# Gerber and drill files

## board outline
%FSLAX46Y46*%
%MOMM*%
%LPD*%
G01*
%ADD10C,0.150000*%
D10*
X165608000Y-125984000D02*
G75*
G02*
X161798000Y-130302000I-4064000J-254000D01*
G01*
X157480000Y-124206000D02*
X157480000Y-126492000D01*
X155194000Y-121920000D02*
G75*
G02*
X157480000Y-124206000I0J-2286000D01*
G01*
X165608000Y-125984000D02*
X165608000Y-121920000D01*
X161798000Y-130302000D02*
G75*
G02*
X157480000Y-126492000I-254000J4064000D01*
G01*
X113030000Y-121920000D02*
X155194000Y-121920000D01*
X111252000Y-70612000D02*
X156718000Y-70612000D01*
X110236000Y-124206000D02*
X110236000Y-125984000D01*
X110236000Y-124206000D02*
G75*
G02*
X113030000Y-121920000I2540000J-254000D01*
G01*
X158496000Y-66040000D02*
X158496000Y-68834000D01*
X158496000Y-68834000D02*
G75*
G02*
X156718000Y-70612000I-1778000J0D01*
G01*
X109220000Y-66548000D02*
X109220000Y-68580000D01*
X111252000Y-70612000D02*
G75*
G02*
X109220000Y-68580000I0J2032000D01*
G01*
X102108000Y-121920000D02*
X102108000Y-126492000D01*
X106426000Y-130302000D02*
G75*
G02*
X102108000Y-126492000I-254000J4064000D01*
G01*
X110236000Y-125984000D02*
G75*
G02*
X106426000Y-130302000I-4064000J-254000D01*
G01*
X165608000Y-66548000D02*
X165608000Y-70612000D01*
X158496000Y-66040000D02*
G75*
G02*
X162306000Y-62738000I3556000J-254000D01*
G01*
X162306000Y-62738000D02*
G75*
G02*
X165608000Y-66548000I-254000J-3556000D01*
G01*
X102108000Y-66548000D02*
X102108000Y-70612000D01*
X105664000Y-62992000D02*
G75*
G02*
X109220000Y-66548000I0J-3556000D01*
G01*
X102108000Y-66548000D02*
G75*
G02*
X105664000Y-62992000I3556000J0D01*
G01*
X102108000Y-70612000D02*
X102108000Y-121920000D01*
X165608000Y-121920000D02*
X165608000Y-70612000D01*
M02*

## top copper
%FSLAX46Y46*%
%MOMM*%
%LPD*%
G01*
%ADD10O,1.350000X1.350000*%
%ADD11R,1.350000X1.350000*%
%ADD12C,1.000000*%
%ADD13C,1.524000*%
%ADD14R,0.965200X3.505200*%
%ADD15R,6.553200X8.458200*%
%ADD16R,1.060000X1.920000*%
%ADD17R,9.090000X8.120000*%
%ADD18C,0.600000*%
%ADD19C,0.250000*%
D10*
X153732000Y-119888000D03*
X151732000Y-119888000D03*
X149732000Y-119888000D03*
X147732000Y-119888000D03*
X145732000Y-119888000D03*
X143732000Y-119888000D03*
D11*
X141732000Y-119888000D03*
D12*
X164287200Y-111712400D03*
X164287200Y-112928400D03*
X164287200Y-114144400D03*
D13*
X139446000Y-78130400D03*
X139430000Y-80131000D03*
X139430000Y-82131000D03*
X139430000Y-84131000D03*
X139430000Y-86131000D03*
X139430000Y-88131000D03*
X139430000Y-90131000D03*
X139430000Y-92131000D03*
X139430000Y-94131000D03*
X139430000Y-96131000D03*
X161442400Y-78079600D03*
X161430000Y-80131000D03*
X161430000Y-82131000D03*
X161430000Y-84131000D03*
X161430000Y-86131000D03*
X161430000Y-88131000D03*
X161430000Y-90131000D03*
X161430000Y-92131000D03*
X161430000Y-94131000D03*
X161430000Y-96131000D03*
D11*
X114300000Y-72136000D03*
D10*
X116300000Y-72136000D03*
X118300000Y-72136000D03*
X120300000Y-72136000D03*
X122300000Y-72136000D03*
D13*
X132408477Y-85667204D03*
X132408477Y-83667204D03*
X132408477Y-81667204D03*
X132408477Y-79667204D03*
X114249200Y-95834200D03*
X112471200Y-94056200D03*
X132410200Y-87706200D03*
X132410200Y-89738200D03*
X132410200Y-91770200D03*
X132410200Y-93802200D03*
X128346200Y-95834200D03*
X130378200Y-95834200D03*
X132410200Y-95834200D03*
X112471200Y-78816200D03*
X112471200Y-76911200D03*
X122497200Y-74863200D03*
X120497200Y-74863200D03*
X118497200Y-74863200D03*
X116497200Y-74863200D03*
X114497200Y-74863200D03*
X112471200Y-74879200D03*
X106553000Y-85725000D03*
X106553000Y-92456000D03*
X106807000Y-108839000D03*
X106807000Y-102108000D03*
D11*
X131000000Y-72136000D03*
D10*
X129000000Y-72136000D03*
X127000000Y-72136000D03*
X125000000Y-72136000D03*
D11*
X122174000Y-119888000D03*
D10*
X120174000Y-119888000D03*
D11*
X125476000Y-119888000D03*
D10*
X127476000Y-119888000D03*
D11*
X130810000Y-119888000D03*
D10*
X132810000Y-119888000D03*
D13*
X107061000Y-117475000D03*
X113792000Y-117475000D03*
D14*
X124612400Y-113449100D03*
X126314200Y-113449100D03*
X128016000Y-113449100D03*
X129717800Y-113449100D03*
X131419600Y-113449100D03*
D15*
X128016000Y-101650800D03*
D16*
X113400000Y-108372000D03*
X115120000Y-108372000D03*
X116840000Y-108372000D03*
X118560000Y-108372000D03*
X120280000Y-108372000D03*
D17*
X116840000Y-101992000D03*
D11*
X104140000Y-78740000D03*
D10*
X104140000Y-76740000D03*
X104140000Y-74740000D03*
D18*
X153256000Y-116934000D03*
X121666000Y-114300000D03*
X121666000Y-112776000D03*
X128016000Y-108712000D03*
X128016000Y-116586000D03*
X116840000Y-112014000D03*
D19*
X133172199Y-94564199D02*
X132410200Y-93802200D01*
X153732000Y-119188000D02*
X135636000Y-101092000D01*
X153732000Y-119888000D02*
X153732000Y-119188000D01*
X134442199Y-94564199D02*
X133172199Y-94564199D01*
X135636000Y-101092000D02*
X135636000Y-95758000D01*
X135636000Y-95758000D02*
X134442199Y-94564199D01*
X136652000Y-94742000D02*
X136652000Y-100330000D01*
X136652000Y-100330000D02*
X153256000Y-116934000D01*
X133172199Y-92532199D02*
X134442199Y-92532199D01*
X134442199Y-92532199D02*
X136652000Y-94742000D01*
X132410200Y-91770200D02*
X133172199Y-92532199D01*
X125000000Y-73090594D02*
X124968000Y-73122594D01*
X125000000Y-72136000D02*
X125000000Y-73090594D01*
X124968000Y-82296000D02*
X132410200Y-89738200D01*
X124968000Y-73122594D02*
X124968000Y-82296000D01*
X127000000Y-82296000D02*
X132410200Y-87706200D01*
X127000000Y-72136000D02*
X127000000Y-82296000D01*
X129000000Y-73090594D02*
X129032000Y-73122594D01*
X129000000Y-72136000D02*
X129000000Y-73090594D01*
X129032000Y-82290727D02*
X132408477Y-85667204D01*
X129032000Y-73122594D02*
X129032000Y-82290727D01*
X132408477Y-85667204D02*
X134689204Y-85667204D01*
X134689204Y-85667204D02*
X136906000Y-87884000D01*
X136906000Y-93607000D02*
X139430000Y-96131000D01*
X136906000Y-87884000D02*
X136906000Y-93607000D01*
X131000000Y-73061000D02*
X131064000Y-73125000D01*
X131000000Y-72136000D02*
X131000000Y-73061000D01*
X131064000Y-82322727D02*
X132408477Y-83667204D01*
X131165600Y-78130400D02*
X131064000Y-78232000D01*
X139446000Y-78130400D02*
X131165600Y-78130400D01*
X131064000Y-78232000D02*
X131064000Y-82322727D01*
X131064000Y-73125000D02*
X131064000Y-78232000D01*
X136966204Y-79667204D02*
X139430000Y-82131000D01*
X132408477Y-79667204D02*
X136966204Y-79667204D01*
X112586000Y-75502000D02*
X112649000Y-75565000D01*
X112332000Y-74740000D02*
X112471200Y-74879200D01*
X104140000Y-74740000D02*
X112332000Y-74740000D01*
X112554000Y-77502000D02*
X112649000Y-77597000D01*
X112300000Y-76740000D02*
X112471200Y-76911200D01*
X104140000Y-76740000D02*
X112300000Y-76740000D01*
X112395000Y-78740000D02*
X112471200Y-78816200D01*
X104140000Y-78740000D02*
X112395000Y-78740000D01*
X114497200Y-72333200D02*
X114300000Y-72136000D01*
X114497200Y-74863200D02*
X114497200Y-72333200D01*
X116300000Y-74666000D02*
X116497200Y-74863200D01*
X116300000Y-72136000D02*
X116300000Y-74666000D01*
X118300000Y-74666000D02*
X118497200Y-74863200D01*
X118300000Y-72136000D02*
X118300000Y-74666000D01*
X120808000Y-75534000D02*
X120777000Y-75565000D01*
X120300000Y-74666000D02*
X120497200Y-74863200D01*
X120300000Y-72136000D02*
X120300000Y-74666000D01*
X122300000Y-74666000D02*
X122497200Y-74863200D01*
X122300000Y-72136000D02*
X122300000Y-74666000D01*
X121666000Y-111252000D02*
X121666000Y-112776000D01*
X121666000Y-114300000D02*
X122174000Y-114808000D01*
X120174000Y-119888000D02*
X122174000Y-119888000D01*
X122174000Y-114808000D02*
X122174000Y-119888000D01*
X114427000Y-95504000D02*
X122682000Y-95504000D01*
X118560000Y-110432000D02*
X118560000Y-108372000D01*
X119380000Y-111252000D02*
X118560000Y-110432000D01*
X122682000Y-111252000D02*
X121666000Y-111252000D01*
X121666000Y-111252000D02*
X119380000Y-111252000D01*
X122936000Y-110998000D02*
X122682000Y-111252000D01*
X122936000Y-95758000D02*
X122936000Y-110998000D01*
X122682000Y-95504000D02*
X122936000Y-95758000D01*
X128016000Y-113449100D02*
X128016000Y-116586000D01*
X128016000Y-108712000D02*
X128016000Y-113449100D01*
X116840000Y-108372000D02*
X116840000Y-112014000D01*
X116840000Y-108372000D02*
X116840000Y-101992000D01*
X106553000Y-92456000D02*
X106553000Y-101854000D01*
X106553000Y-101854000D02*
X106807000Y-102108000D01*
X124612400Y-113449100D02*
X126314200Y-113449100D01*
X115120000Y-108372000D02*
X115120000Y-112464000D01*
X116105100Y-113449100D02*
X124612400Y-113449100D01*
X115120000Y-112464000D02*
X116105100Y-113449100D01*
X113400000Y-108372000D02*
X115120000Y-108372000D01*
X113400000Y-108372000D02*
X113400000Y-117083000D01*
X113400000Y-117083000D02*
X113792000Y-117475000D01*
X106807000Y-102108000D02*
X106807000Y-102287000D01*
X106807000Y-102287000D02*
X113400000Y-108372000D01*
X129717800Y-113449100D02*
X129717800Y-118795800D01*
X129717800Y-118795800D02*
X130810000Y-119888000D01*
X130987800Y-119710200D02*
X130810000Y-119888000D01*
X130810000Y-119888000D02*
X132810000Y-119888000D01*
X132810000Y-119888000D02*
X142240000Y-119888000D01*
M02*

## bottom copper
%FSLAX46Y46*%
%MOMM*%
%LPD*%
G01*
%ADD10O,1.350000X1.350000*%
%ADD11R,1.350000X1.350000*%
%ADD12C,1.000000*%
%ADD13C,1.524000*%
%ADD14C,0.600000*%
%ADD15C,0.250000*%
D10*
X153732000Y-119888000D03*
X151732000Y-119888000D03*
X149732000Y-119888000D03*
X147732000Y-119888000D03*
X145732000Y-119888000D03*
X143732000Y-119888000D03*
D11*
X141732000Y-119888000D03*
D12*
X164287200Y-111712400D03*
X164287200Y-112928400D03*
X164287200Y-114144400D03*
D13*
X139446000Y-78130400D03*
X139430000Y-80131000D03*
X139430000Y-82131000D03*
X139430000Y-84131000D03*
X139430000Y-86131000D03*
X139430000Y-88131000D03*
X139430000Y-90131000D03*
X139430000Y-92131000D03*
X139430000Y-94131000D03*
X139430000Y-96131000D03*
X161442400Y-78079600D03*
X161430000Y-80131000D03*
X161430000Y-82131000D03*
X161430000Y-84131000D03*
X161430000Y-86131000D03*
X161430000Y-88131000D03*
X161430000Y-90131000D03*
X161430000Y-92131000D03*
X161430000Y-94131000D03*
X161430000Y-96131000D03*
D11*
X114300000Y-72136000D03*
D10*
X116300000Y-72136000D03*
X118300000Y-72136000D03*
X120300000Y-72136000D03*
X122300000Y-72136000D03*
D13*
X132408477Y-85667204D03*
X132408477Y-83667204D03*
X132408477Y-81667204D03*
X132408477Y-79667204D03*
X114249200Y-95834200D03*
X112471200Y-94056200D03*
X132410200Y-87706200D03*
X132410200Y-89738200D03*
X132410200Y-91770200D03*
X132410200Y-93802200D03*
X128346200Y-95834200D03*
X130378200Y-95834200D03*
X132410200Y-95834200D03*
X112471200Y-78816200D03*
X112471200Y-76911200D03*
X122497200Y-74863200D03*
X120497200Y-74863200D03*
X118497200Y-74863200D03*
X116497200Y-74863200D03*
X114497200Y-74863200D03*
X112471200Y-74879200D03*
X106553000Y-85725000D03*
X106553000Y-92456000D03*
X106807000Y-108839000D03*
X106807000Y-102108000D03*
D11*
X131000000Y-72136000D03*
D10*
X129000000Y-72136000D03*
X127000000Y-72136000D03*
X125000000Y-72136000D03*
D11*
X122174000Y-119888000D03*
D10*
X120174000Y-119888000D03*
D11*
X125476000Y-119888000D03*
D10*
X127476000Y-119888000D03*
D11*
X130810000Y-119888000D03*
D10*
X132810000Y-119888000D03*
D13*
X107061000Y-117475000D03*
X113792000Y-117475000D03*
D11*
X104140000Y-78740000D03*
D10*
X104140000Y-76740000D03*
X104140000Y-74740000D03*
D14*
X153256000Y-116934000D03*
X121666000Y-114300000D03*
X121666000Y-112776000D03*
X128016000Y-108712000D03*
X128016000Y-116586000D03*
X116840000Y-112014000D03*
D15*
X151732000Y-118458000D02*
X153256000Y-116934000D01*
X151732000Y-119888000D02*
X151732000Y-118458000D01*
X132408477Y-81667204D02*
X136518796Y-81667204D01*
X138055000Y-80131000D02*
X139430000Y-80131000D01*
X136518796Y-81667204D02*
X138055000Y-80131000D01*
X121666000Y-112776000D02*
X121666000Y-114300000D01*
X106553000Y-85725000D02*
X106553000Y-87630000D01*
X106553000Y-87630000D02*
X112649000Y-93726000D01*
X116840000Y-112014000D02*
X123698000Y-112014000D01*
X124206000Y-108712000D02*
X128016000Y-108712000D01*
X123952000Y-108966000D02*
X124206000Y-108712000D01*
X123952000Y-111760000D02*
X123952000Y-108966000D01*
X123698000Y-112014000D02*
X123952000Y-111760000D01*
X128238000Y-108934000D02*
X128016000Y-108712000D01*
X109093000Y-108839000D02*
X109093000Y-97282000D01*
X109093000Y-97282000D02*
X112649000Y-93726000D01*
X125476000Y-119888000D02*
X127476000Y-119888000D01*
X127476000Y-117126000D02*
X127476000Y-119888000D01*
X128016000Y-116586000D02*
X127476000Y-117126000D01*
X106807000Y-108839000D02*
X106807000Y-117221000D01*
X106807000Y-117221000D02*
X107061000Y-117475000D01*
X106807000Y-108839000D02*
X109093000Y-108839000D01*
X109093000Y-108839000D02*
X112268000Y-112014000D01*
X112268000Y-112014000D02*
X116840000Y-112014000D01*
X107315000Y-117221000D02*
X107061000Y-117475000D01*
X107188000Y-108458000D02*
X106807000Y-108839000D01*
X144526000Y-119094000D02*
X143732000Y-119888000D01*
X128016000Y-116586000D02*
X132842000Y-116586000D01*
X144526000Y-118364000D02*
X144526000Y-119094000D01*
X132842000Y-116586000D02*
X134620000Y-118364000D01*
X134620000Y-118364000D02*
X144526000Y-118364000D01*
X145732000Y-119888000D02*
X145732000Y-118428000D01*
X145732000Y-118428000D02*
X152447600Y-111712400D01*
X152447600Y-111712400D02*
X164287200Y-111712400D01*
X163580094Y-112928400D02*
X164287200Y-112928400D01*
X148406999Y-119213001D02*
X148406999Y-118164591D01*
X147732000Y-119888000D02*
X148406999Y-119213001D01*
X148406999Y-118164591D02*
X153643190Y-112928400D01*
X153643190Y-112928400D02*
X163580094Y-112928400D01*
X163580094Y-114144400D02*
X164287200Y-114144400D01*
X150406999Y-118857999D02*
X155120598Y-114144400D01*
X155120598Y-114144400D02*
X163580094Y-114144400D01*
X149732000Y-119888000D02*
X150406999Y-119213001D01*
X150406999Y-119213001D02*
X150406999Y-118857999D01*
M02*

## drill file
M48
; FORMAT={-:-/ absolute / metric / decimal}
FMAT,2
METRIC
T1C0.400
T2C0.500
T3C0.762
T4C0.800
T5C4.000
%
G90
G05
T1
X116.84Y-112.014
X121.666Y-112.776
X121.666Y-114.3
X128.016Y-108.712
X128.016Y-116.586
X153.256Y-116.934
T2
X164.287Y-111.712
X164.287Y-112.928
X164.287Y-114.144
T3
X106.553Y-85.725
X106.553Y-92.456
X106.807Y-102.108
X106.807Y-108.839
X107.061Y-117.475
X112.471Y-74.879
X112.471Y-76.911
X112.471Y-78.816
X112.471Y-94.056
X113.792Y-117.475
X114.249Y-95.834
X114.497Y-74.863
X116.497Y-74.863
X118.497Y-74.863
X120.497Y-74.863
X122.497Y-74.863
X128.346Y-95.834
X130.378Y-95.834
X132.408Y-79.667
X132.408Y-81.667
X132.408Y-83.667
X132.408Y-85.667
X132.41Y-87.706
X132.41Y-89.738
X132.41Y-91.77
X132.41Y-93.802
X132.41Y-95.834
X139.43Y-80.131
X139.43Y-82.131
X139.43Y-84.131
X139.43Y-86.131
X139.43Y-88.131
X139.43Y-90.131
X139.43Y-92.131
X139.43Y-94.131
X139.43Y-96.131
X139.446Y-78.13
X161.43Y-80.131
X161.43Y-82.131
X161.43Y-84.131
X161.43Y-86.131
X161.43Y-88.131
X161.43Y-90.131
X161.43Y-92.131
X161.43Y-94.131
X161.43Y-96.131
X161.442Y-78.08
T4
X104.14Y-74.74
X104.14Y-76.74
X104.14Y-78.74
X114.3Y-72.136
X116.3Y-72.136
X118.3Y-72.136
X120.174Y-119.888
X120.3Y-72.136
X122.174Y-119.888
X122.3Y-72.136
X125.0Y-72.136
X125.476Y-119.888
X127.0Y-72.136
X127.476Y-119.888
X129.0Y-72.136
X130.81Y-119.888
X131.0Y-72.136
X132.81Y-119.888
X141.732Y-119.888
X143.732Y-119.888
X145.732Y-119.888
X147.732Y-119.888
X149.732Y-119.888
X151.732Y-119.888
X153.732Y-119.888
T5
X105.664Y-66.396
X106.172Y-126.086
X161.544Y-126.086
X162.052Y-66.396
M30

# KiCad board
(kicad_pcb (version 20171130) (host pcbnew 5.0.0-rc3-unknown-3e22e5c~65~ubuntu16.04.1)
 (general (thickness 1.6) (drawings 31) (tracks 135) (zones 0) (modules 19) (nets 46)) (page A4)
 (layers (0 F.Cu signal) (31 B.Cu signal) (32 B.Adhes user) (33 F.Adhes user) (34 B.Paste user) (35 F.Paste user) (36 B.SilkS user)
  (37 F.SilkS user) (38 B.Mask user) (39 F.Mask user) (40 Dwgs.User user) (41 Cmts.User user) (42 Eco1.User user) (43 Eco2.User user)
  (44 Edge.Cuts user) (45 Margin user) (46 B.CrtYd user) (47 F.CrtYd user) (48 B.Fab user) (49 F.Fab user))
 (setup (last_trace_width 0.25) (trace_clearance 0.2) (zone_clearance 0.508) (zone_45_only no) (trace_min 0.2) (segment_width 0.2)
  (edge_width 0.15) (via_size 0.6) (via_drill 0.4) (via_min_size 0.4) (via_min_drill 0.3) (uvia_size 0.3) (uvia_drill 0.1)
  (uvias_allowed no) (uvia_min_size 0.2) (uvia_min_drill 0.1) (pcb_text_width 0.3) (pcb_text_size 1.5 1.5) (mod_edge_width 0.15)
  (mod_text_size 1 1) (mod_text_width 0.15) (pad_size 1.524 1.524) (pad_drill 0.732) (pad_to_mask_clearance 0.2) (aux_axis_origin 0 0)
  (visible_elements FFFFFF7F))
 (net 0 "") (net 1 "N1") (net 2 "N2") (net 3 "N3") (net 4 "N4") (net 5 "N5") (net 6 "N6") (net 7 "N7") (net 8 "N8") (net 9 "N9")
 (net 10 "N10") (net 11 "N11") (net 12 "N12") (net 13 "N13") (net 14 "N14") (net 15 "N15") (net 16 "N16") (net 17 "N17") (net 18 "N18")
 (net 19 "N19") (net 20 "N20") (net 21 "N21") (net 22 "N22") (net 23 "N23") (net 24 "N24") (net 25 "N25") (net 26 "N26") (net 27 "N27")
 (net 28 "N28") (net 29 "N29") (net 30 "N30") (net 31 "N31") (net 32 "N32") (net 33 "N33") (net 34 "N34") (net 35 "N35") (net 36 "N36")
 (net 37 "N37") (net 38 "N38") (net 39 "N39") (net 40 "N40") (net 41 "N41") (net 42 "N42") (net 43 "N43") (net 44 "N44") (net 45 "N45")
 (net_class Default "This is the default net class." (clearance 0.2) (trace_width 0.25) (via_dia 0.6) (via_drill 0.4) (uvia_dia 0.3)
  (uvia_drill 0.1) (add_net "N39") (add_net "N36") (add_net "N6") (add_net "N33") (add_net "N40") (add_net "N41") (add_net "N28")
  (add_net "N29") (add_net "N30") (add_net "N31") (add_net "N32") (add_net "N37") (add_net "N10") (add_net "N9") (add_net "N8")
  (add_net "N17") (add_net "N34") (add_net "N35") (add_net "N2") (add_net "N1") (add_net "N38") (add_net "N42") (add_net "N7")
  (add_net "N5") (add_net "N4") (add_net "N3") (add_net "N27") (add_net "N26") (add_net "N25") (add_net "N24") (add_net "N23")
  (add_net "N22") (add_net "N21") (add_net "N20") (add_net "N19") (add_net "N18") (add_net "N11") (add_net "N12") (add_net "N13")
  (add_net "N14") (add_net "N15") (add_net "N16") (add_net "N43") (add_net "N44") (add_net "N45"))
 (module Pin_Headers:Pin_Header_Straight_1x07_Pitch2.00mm (layer F.Cu) (at 141.732 119.888 90)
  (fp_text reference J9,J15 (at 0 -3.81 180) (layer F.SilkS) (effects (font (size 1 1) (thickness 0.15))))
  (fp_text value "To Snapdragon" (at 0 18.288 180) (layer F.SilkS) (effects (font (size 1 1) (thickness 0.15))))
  (pad 7 thru_hole oval (at 0 12 90) (size 1.35 1.35) (drill 0.8) (layers *.Cu *.Mask) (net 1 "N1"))
  (pad 6 thru_hole oval (at 0 10 90) (size 1.35 1.35) (drill 0.8) (layers *.Cu *.Mask) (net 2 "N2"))
  (pad 5 thru_hole oval (at 0 8 90) (size 1.35 1.35) (drill 0.8) (layers *.Cu *.Mask) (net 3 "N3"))
  (pad 4 thru_hole oval (at 0 6 90) (size 1.35 1.35) (drill 0.8) (layers *.Cu *.Mask) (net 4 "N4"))
  (pad 3 thru_hole oval (at 0 4 90) (size 1.35 1.35) (drill 0.8) (layers *.Cu *.Mask) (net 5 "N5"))
  (pad 2 thru_hole oval (at 0 2 90) (size 1.35 1.35) (drill 0.8) (layers *.Cu *.Mask) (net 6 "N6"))
  (pad 1 thru_hole rect (at 0 0 90) (size 1.35 1.35) (drill 0.8) (layers *.Cu *.Mask) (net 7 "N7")))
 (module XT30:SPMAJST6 (layer F.Cu) (at 163.576 113.792 270)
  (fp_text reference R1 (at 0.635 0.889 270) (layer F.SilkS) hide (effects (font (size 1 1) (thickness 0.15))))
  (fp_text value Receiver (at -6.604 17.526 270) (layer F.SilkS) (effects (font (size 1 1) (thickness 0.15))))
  (pad 1 thru_hole circle (at -2.0796 -0.7112 270) (size 1 1) (drill 0.5) (layers *.Cu *.Mask) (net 5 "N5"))
  (pad 2 thru_hole circle (at -0.8636 -0.7112 270) (size 1 1) (drill 0.5) (layers *.Cu *.Mask) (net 4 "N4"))
  (pad 3 thru_hole circle (at 0.3524 -0.7112 270) (size 1 1) (drill 0.5) (layers *.Cu *.Mask) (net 3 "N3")))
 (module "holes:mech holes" (layer F.Cu) (at 162.052 129.286)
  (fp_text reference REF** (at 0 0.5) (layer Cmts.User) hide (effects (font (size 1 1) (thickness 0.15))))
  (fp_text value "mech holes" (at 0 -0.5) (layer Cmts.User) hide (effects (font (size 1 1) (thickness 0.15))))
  (pad "" np_thru_hole circle (at -0.508 -3.2004) (size 4 4) (drill 4) (layers *.Cu *.Mask)))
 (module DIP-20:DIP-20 (layer F.Cu) (at 138.176 104.14)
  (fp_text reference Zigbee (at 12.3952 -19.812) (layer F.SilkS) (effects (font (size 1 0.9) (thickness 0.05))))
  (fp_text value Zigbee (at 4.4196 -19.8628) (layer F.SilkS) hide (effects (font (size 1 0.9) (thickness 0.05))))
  (pad 1 thru_hole circle (at 1.27 -26.0096) (size 1.524 1.524) (drill 0.762) (layers *.Cu *.Mask F.SilkS) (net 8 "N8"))
  (pad 2 thru_hole circle (at 1.254 -24.009) (size 1.524 1.524) (drill 0.762) (layers *.Cu *.Mask F.SilkS) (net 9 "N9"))
  (pad 3 thru_hole circle (at 1.254 -22.009) (size 1.524 1.524) (drill 0.762) (layers *.Cu *.Mask F.SilkS) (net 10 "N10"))
  (pad 4 thru_hole circle (at 1.254 -20.009) (size 1.524 1.524) (drill 0.762) (layers *.Cu *.Mask F.SilkS) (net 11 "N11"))
  (pad 5 thru_hole circle (at 1.254 -18.009) (size 1.524 1.524) (drill 0.762) (layers *.Cu *.Mask F.SilkS) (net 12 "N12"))
  (pad 6 thru_hole circle (at 1.254 -16.009) (size 1.524 1.524) (drill 0.762) (layers *.Cu *.Mask F.SilkS) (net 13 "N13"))
  (pad 7 thru_hole circle (at 1.254 -14.009) (size 1.524 1.524) (drill 0.762) (layers *.Cu *.Mask F.SilkS) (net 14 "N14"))
  (pad 8 thru_hole circle (at 1.254 -12.009) (size 1.524 1.524) (drill 0.762) (layers *.Cu *.Mask F.SilkS) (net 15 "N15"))
  (pad 9 thru_hole circle (at 1.254 -10.009) (size 1.524 1.524) (drill 0.762) (layers *.Cu *.Mask F.SilkS) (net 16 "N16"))
  (pad 10 thru_hole circle (at 1.254 -8.009) (size 1.524 1.524) (drill 0.762) (layers *.Cu *.Mask F.SilkS) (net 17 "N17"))
  (pad 20 thru_hole circle (at 23.2664 -26.0604) (size 1.524 1.524) (drill 0.762) (layers *.Cu *.Mask F.SilkS) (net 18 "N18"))
  (pad 19 thru_hole circle (at 23.254 -24.009) (size 1.524 1.524) (drill 0.762) (layers *.Cu *.Mask F.SilkS) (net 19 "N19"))
  (pad 18 thru_hole circle (at 23.254 -22.009) (size 1.524 1.524) (drill 0.762) (layers *.Cu *.Mask F.SilkS) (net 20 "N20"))
  (pad 17 thru_hole circle (at 23.254 -20.009) (size 1.524 1.524) (drill 0.762) (layers *.Cu *.Mask F.SilkS) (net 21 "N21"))
  (pad 16 thru_hole circle (at 23.254 -18.009) (size 1.524 1.524) (drill 0.762) (layers *.Cu *.Mask F.SilkS) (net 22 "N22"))
  (pad 15 thru_hole circle (at 23.254 -16.009) (size 1.524 1.524) (drill 0.762) (layers *.Cu *.Mask F.SilkS) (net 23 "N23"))
  (pad 14 thru_hole circle (at 23.254 -14.009) (size 1.524 1.524) (drill 0.762) (layers *.Cu *.Mask F.SilkS) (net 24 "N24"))
  (pad 13 thru_hole circle (at 23.254 -12.009) (size 1.524 1.524) (drill 0.762) (layers *.Cu *.Mask F.SilkS) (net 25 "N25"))
  (pad 12 thru_hole circle (at 23.254 -10.009) (size 1.524 1.524) (drill 0.762) (layers *.Cu *.Mask F.SilkS) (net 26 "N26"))
  (pad 11 thru_hole circle (at 23.254 -8.009) (size 1.524 1.524) (drill 0.762) (layers *.Cu *.Mask F.SilkS) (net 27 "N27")))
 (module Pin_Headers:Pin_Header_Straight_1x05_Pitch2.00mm (layer F.Cu) (at 114.3 72.136 90)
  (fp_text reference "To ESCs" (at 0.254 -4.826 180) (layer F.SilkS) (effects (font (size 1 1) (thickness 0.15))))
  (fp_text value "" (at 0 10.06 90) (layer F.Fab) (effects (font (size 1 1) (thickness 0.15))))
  (pad 1 thru_hole rect (at 0 0 90) (size 1.35 1.35) (drill 0.8) (layers *.Cu *.Mask) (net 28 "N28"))
  (pad 2 thru_hole oval (at 0 2 90) (size 1.35 1.35) (drill 0.8) (layers *.Cu *.Mask) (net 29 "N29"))
  (pad 3 thru_hole oval (at 0 4 90) (size 1.35 1.35) (drill 0.8) (layers *.Cu *.Mask) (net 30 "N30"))
  (pad 4 thru_hole oval (at 0 6 90) (size 1.35 1.35) (drill 0.8) (layers *.Cu *.Mask) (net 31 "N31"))
  (pad 5 thru_hole oval (at 0 8 90) (size 1.35 1.35) (drill 0.8) (layers *.Cu *.Mask) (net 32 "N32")))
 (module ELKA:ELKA (layer F.Cu) (at 121.666 85.852)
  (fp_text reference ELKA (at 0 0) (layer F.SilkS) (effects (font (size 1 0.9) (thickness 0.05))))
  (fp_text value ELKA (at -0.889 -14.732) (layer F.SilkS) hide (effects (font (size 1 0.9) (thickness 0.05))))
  (pad D thru_hole circle (at 10.742477 -0.184796) (size 1.524 1.524) (drill 0.762) (layers *.Cu *.Mask B.SilkS) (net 17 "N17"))
  (pad C thru_hole circle (at 10.742477 -2.184796) (size 1.524 1.524) (drill 0.762) (layers *.Cu *.Mask B.SilkS) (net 8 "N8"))
  (pad B thru_hole circle (at 10.742477 -4.184796) (size 1.524 1.524) (drill 0.762) (layers *.Cu *.Mask B.SilkS) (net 9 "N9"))
  (pad A thru_hole circle (at 10.742477 -6.184796) (size 1.524 1.524) (drill 0.762) (layers *.Cu *.Mask B.SilkS) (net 10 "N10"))
  (pad 12 thru_hole circle (at -7.4168 9.9822) (size 1.524 1.524) (drill 0.762) (layers *.Cu *.Mask B.SilkS) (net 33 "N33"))
  (pad 11 thru_hole circle (at -9.1948 8.2042 270) (size 1.524 1.524) (drill 0.762) (layers *.Cu *.Mask B.SilkS) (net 6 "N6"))
  (pad E thru_hole circle (at 10.7442 1.8542 270) (size 1.524 1.524) (drill 0.762) (layers *.Cu *.Mask B.SilkS) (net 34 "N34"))
  (pad F thru_hole circle (at 10.7442 3.8862 270) (size 1.524 1.524) (drill 0.762) (layers *.Cu *.Mask B.SilkS) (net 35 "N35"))
  (pad G thru_hole circle (at 10.7442 5.9182 270) (size 1.524 1.524) (drill 0.762) (layers *.Cu *.Mask B.SilkS) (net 2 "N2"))
  (pad H thru_hole circle (at 10.7442 7.9502 270) (size 1.524 1.524) (drill 0.762) (layers *.Cu *.Mask B.SilkS) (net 1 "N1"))
  (pad 10 thru_hole circle (at 6.6802 9.9822 270) (size 1.524 1.524) (drill 0.762) (layers *.Cu *.Mask B.SilkS) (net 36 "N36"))
  (pad 9 thru_hole circle (at 8.7122 9.9822 270) (size 1.524 1.524) (drill 0.762) (layers *.Cu *.Mask B.SilkS) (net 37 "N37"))
  (pad I thru_hole circle (at 10.7442 9.9822 270) (size 1.524 1.524) (drill 0.762) (layers *.Cu *.Mask B.SilkS) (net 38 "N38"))
  (pad 1 thru_hole circle (at -9.1948 -7.0358 270) (size 1.524 1.524) (drill 0.762) (layers *.Cu *.Mask B.SilkS) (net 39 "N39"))
  (pad 2 thru_hole circle (at -9.1948 -8.9408 270) (size 1.524 1.524) (drill 0.762) (layers *.Cu *.Mask B.SilkS) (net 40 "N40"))
  (pad 8 thru_hole circle (at 0.8312 -10.9888 270) (size 1.524 1.524) (drill 0.762) (layers *.Cu *.Mask B.SilkS) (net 32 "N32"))
  (pad 7 thru_hole circle (at -1.1688 -10.9888 270) (size 1.524 1.524) (drill 0.762) (layers *.Cu *.Mask B.SilkS) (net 31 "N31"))
  (pad 6 thru_hole circle (at -3.1688 -10.9888 270) (size 1.524 1.524) (drill 0.762) (layers *.Cu *.Mask B.SilkS) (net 30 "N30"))
  (pad 5 thru_hole circle (at -5.1688 -10.9888 270) (size 1.524 1.524) (drill 0.762) (layers *.Cu *.Mask B.SilkS) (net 29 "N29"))
  (pad 4 thru_hole circle (at -7.1688 -10.9888 270) (size 1.524 1.524) (drill 0.762) (layers *.Cu *.Mask B.SilkS) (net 28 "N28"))
  (pad 3 thru_hole circle (at -9.1948 -10.9728 270) (size 1.524 1.524) (drill 0.762) (layers *.Cu *.Mask B.SilkS) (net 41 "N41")))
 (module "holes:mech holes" (layer F.Cu) (at 106.172 69.596)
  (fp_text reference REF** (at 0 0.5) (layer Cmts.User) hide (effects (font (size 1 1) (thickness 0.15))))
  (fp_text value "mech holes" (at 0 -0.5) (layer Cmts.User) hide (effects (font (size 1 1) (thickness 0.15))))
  (pad "" np_thru_hole circle (at -0.508 -3.2004) (size 4 4) (drill 4) (layers *.Cu *.Mask)))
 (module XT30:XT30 (layer F.Cu) (at 112.522 87.122 270)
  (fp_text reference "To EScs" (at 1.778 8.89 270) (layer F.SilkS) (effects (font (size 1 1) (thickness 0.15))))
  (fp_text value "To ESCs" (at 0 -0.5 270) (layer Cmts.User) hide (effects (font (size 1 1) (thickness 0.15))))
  (pad 1 thru_hole circle (at -1.397 5.969 270) (size 1.524 1.524) (drill 0.762) (layers *.Cu *.Mask) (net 6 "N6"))
  (pad 2 thru_hole circle (at 5.334 5.969 270) (size 1.524 1.524) (drill 0.762) (layers *.Cu *.Mask) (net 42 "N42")))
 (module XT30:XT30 (layer F.Cu) (at 100.838 107.442 90)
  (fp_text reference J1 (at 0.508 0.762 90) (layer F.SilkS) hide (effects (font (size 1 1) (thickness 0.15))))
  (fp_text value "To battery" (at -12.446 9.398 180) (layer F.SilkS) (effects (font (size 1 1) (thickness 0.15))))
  (pad 1 thru_hole circle (at -1.397 5.969 90) (size 1.524 1.524) (drill 0.762) (layers *.Cu *.Mask) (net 6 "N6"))
  (pad 2 thru_hole circle (at 5.334 5.969 90) (size 1.524 1.524) (drill 0.762) (layers *.Cu *.Mask) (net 42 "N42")))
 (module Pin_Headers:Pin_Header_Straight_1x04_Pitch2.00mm (layer F.Cu) (at 131 72.136 270)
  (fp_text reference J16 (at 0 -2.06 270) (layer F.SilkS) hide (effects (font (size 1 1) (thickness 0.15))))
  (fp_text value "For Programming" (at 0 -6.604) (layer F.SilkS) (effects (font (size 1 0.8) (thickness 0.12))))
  (pad 1 thru_hole rect (at 0 0 270) (size 1.35 1.35) (drill 0.8) (layers *.Cu *.Mask) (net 8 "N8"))
  (pad 2 thru_hole oval (at 0 2 270) (size 1.35 1.35) (drill 0.8) (layers *.Cu *.Mask) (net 17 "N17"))
  (pad 3 thru_hole oval (at 0 4 270) (size 1.35 1.35) (drill 0.8) (layers *.Cu *.Mask) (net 34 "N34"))
  (pad 4 thru_hole oval (at 0 6 270) (size 1.35 1.35) (drill 0.8) (layers *.Cu *.Mask) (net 35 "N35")))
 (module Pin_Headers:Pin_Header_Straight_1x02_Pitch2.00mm (layer F.Cu) (at 122.174 119.888 270)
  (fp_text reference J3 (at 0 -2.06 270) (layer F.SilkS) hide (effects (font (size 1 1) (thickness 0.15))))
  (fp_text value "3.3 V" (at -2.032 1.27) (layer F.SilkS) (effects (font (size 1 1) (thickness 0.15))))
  (pad 1 thru_hole rect (at 0 0 270) (size 1.35 1.35) (drill 0.8) (layers *.Cu *.Mask) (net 33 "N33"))
  (pad 2 thru_hole oval (at 0 2 270) (size 1.35 1.35) (drill 0.8) (layers *.Cu *.Mask) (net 33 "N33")))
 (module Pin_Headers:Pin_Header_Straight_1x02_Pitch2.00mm (layer F.Cu) (at 125.476 119.888 90)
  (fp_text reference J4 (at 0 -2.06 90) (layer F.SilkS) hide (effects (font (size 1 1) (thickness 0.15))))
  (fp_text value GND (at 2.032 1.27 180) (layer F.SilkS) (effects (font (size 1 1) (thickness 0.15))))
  (pad 1 thru_hole rect (at 0 0 90) (size 1.35 1.35) (drill 0.8) (layers *.Cu *.Mask) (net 6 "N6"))
  (pad 2 thru_hole oval (at 0 2 90) (size 1.35 1.35) (drill 0.8) (layers *.Cu *.Mask) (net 6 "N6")))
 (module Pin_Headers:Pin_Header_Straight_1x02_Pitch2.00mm (layer F.Cu) (at 130.81 119.888 90)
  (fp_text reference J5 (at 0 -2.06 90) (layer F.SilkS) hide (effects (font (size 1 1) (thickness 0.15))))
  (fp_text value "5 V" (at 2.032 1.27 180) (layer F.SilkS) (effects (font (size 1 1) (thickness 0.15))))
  (pad 1 thru_hole rect (at 0 0 90) (size 1.35 1.35) (drill 0.8) (layers *.Cu *.Mask) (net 7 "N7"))
  (pad 2 thru_hole oval (at 0 2 90) (size 1.35 1.35) (drill 0.8) (layers *.Cu *.Mask) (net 7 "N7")))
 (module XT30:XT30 (layer F.Cu) (at 108.458 111.506)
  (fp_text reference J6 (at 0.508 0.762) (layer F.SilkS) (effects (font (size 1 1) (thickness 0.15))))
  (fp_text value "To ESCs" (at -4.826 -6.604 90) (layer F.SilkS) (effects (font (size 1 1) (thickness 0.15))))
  (pad 1 thru_hole circle (at -1.397 5.969) (size 1.524 1.524) (drill 0.762) (layers *.Cu *.Mask) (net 6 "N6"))
  (pad 2 thru_hole circle (at 5.334 5.969) (size 1.524 1.524) (drill 0.762) (layers *.Cu *.Mask) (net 42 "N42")))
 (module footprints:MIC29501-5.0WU (layer F.Cu) (at 128.016 104.394)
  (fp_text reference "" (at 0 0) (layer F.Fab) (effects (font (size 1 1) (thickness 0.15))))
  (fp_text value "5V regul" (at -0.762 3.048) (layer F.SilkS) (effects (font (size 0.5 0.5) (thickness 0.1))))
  (pad 1 smd rect (at -3.4036 9.0551) (size 0.9652 3.5052) (layers F.Cu F.Paste F.Mask) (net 42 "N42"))
  (pad 2 smd rect (at -1.7018 9.0551) (size 0.9652 3.5052) (layers F.Cu F.Paste F.Mask) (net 42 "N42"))
  (pad 3 smd rect (at 0 9.0551) (size 0.9652 3.5052) (layers F.Cu F.Paste F.Mask) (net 6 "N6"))
  (pad 4 smd rect (at 1.7018 9.0551) (size 0.9652 3.5052) (layers F.Cu F.Paste F.Mask) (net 7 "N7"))
  (pad 5 smd rect (at 3.4036 9.0551) (size 0.9652 3.5052) (layers F.Cu F.Paste F.Mask) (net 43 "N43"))
  (pad 6 smd rect (at 0 -2.7432) (size 6.5532 8.4582) (layers F.Cu F.Paste F.Mask) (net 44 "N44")))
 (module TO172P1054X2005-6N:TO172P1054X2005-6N (layer F.Cu) (at 116.84 103.632)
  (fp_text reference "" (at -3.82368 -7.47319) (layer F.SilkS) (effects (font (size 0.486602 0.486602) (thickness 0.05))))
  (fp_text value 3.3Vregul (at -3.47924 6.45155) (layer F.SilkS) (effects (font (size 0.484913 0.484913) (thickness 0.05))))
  (pad 1 smd rect (at -3.44 4.74 90) (size 1.92 1.06) (layers F.Cu F.Paste F.Mask) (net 42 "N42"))
  (pad 2 smd rect (at -1.72 4.74 90) (size 1.92 1.06) (layers F.Cu F.Paste F.Mask) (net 42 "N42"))
  (pad 3 smd rect (at 0 4.74 90) (size 1.92 1.06) (layers F.Cu F.Paste F.Mask) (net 6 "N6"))
  (pad 4 smd rect (at 1.72 4.74 90) (size 1.92 1.06) (layers F.Cu F.Paste F.Mask) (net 33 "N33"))
  (pad 5 smd rect (at 3.44 4.74 90) (size 1.92 1.06) (layers F.Cu F.Paste F.Mask) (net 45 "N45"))
  (pad 6 smd rect (at 0 -1.64 90) (size 8.12 9.09) (layers F.Cu F.Paste F.Mask) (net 6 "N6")))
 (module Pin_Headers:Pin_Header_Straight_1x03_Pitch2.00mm (layer F.Cu) (at 104.14 78.74 180)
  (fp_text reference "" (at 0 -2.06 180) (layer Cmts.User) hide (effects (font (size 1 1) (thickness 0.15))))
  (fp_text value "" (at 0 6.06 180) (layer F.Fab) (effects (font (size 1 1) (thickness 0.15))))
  (pad 1 thru_hole rect (at 0 0 180) (size 1.35 1.35) (drill 0.8) (layers *.Cu *.Mask) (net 39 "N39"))
  (pad 2 thru_hole oval (at 0 2 180) (size 1.35 1.35) (drill 0.8) (layers *.Cu *.Mask) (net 40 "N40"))
  (pad 3 thru_hole oval (at 0 4 180) (size 1.35 1.35) (drill 0.8) (layers *.Cu *.Mask) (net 41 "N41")))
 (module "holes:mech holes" (layer F.Cu) (at 162.56 69.596)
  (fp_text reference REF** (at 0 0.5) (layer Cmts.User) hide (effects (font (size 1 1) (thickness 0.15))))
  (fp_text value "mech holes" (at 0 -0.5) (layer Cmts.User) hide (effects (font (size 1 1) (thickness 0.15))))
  (pad "" np_thru_hole circle (at -0.508 -3.2004) (size 4 4) (drill 4) (layers *.Cu *.Mask)))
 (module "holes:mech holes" (layer F.Cu) (at 106.68 129.286)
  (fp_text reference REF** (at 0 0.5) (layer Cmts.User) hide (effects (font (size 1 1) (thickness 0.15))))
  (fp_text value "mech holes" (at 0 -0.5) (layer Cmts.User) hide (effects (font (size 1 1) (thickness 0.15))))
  (pad "" np_thru_hole circle (at -0.508 -3.2004) (size 4 4) (drill 4) (layers *.Cu *.Mask)))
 (gr_arc (start 161.544 126.238) (end 165.608 125.984) (angle 90) (layer Edge.Cuts) (width 0.15))
 (gr_line (start 157.48 124.206) (end 157.48 126.492) (angle 90) (layer Edge.Cuts) (width 0.15))
 (gr_arc (start 155.194 124.206) (end 155.194 121.92) (angle 90) (layer Edge.Cuts) (width 0.15))
 (gr_line (start 165.608 125.984) (end 165.608 121.92) (angle 90) (layer Edge.Cuts) (width 0.15))
 (gr_arc (start 161.544 126.238) (end 161.798 130.302) (angle 90) (layer Edge.Cuts) (width 0.15))
 (gr_line (start 113.03 121.92) (end 155.194 121.92) (angle 90) (layer Edge.Cuts) (width 0.15))
 (gr_line (start 111.252 70.612) (end 156.718 70.612) (angle 90) (layer Edge.Cuts) (width 0.15))
 (gr_line (start 110.236 124.206) (end 110.236 125.984) (angle 90) (layer Edge.Cuts) (width 0.15))
 (gr_arc (start 112.776 124.46) (end 110.236 124.206) (angle 90) (layer Edge.Cuts) (width 0.15))
 (gr_line (start 158.496 66.04) (end 158.496 68.834) (angle 90) (layer Edge.Cuts) (width 0.15))
 (gr_arc (start 156.718 68.834) (end 158.496 68.834) (angle 90) (layer Edge.Cuts) (width 0.15))
 (gr_line (start 109.22 66.548) (end 109.22 68.58) (angle 90) (layer Edge.Cuts) (width 0.15))
 (gr_arc (start 111.252 68.58) (end 111.252 70.612) (angle 90) (layer Edge.Cuts) (width 0.15))
 (gr_line (start 102.108 121.92) (end 102.108 126.492) (angle 90) (layer Edge.Cuts) (width 0.15))
 (gr_arc (start 106.172 126.238) (end 106.426 130.302) (angle 90) (layer Edge.Cuts) (width 0.15))
 (gr_arc (start 106.172 126.238) (end 110.236 125.984) (angle 90) (layer Edge.Cuts) (width 0.15))
 (gr_line (start 165.608 66.548) (end 165.608 70.612) (angle 90) (layer Edge.Cuts) (width 0.15))
 (gr_arc (start 162.052 66.294) (end 158.496 66.04) (angle 90) (layer Edge.Cuts) (width 0.15))
 (gr_arc (start 162.052 66.294) (end 162.306 62.738) (angle 90) (layer Edge.Cuts) (width 0.15))
 (gr_line (start 102.108 66.548) (end 102.108 70.612) (angle 90) (layer Edge.Cuts) (width 0.15))
 (gr_arc (start 105.664 66.548) (end 105.664 62.992) (angle 90) (layer Edge.Cuts) (width 0.15))
 (gr_arc (start 105.664 66.548) (end 102.108 66.548) (angle 90) (layer Edge.Cuts) (width 0.15))
 (gr_line (start 102.108 70.612) (end 102.108 121.92) (angle 90) (layer Edge.Cuts) (width 0.15))
 (gr_line (start 165.608 121.92) (end 165.608 70.612) (angle 90) (layer Edge.Cuts) (width 0.15))
 (segment (start 133.172199 94.564199) (end 132.4102 93.8022) (width 0.25) (layer F.Cu) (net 1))
 (segment (start 153.732 119.188) (end 135.636 101.092) (width 0.25) (layer F.Cu) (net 1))
 (segment (start 153.732 119.888) (end 153.732 119.188) (width 0.25) (layer F.Cu) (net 1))
 (segment (start 134.442199 94.564199) (end 133.172199 94.564199) (width 0.25) (layer F.Cu) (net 1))
 (segment (start 135.636 101.092) (end 135.636 95.758) (width 0.25) (layer F.Cu) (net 1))
 (segment (start 135.636 95.758) (end 134.442199 94.564199) (width 0.25) (layer F.Cu) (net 1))
 (segment (start 136.652 94.742) (end 136.652 100.33) (width 0.25) (layer F.Cu) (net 2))
 (segment (start 136.652 100.33) (end 153.256 116.934) (width 0.25) (layer F.Cu) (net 2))
 (segment (start 133.172199 92.532199) (end 134.442199 92.532199) (width 0.25) (layer F.Cu) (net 2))
 (segment (start 134.442199 92.532199) (end 136.652 94.742) (width 0.25) (layer F.Cu) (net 2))
 (segment (start 132.4102 91.7702) (end 133.172199 92.532199) (width 0.25) (layer F.Cu) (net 2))
 (via (at 153.256 116.934) (size 0.6) (drill 0.4) (layers F.Cu B.Cu) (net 2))
 (segment (start 151.732 118.458) (end 153.256 116.934) (width 0.25) (layer B.Cu) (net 2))
 (segment (start 151.732 119.888) (end 151.732 118.458) (width 0.25) (layer B.Cu) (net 2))
 (segment (start 125 73.090594) (end 124.968 73.122594) (width 0.25) (layer F.Cu) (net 35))
 (segment (start 125 72.136) (end 125 73.090594) (width 0.25) (layer F.Cu) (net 35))
 (segment (start 124.968 82.296) (end 132.4102 89.7382) (width 0.25) (layer F.Cu) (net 35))
 (segment (start 124.968 73.122594) (end 124.968 82.296) (width 0.25) (layer F.Cu) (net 35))
 (segment (start 127 82.296) (end 132.4102 87.7062) (width 0.25) (layer F.Cu) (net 34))
 (segment (start 127 72.136) (end 127 82.296) (width 0.25) (layer F.Cu) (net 34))
 (segment (start 129 73.090594) (end 129.032 73.122594) (width 0.25) (layer F.Cu) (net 17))
 (segment (start 129 72.136) (end 129 73.090594) (width 0.25) (layer F.Cu) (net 17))
 (segment (start 129.032 82.290727) (end 132.408477 85.667204) (width 0.25) (layer F.Cu) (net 17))
 (segment (start 129.032 73.122594) (end 129.032 82.290727) (width 0.25) (layer F.Cu) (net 17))
 (segment (start 132.408477 85.667204) (end 134.689204 85.667204) (width 0.25) (layer F.Cu) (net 17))
 (segment (start 134.689204 85.667204) (end 136.906 87.884) (width 0.25) (layer F.Cu) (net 17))
 (segment (start 136.906 93.607) (end 139.43 96.131) (width 0.25) (layer F.Cu) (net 17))
 (segment (start 136.906 87.884) (end 136.906 93.607) (width 0.25) (layer F.Cu) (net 17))
 (segment (start 131 73.061) (end 131.064 73.125) (width 0.25) (layer F.Cu) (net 8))
 (segment (start 131 72.136) (end 131 73.061) (width 0.25) (layer F.Cu) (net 8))
 (segment (start 131.064 82.322727) (end 132.408477 83.667204) (width 0.25) (layer F.Cu) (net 8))
 (segment (start 131.1656 78.1304) (end 131.064 78.232) (width 0.25) (layer F.Cu) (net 8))
 (segment (start 139.446 78.1304) (end 131.1656 78.1304) (width 0.25) (layer F.Cu) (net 8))
 (segment (start 131.064 78.232) (end 131.064 82.322727) (width 0.25) (layer F.Cu) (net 8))
 (segment (start 131.064 73.125) (end 131.064 78.232) (width 0.25) (layer F.Cu) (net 8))
 (segment (start 132.408477 81.667204) (end 136.518796 81.667204) (width 0.25) (layer B.Cu) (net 9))
 (segment (start 138.055 80.131) (end 139.43 80.131) (width 0.25) (layer B.Cu) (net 9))
 (segment (start 136.518796 81.667204) (end 138.055 80.131) (width 0.25) (layer B.Cu) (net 9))
 (segment (start 136.966204 79.667204) (end 139.43 82.131) (width 0.25) (layer F.Cu) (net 10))
 (segment (start 132.408477 79.667204) (end 136.966204 79.667204) (width 0.25) (layer F.Cu) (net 10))
 (segment (start 112.586 75.502) (end 112.649 75.565) (width 0.25) (layer F.Cu) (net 41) (status 30))
 (segment (start 112.332 74.74) (end 112.4712 74.8792) (width 0.25) (layer F.Cu) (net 41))
 (segment (start 104.14 74.74) (end 112.332 74.74) (width 0.25) (layer F.Cu) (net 41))
 (segment (start 112.554 77.502) (end 112.649 77.597) (width 0.25) (layer F.Cu) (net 40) (status 30))
 (segment (start 112.3 76.74) (end 112.4712 76.9112) (width 0.25) (layer F.Cu) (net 40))
 (segment (start 104.14 76.74) (end 112.3 76.74) (width 0.25) (layer F.Cu) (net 40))
 (segment (start 112.395 78.74) (end 112.4712 78.8162) (width 0.25) (layer F.Cu) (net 39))
 (segment (start 104.14 78.74) (end 112.395 78.74) (width 0.25) (layer F.Cu) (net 39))
 (segment (start 114.4972 72.3332) (end 114.3 72.136) (width 0.25) (layer F.Cu) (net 28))
 (segment (start 114.4972 74.8632) (end 114.4972 72.3332) (width 0.25) (layer F.Cu) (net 28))
 (segment (start 116.3 74.666) (end 116.4972 74.8632) (width 0.25) (layer F.Cu) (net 29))
 (segment (start 116.3 72.136) (end 116.3 74.666) (width 0.25) (layer F.Cu) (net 29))
 (segment (start 118.3 74.666) (end 118.4972 74.8632) (width 0.25) (layer F.Cu) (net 30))
 (segment (start 118.3 72.136) (end 118.3 74.666) (width 0.25) (layer F.Cu) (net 30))
 (segment (start 120.808 75.534) (end 120.777 75.565) (width 0.25) (layer F.Cu) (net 31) (status 30))
 (segment (start 120.3 74.666) (end 120.4972 74.8632) (width 0.25) (layer F.Cu) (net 31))
 (segment (start 120.3 72.136) (end 120.3 74.666) (width 0.25) (layer F.Cu) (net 31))
 (segment (start 122.3 74.666) (end 122.4972 74.8632) (width 0.25) (layer F.Cu) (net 32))
 (segment (start 122.3 72.136) (end 122.3 74.666) (width 0.25) (layer F.Cu) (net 32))
 (segment (start 121.666 111.252) (end 121.666 112.776) (width 0.25) (layer F.Cu) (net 33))
 (segment (start 121.666 114.3) (end 122.174 114.808) (width 0.25) (layer F.Cu) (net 33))
 (via (at 121.666 114.3) (size 0.6) (drill 0.4) (layers F.Cu B.Cu) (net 33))
 (segment (start 121.666 112.776) (end 121.666 114.3) (width 0.25) (layer B.Cu) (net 33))
 (via (at 121.666 112.776) (size 0.6) (drill 0.4) (layers F.Cu B.Cu) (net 33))
 (segment (start 120.174 119.888) (end 122.174 119.888) (width 0.25) (layer F.Cu) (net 33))
 (segment (start 122.174 114.808) (end 122.174 119.888) (width 0.25) (layer F.Cu) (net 33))
 (segment (start 114.427 95.504) (end 122.682 95.504) (width 0.25) (layer F.Cu) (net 33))
 (segment (start 118.56 110.432) (end 118.56 108.372) (width 0.25) (layer F.Cu) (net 33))
 (segment (start 119.38 111.252) (end 118.56 110.432) (width 0.25) (layer F.Cu) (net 33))
 (segment (start 122.682 111.252) (end 121.666 111.252) (width 0.25) (layer F.Cu) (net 33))
 (segment (start 121.666 111.252) (end 119.38 111.252) (width 0.25) (layer F.Cu) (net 33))
 (segment (start 122.936 110.998) (end 122.682 111.252) (width 0.25) (layer F.Cu) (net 33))
 (segment (start 122.936 95.758) (end 122.936 110.998) (width 0.25) (layer F.Cu) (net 33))
 (segment (start 122.682 95.504) (end 122.936 95.758) (width 0.25) (layer F.Cu) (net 33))
 (segment (start 106.553 85.725) (end 106.553 87.63) (width 0.25) (layer B.Cu) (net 6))
 (segment (start 106.553 87.63) (end 112.649 93.726) (width 0.25) (layer B.Cu) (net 6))
 (segment (start 116.84 112.014) (end 123.698 112.014) (width 0.25) (layer B.Cu) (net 6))
 (segment (start 124.206 108.712) (end 128.016 108.712) (width 0.25) (layer B.Cu) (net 6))
 (segment (start 123.952 108.966) (end 124.206 108.712) (width 0.25) (layer B.Cu) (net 6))
 (segment (start 123.952 111.76) (end 123.952 108.966) (width 0.25) (layer B.Cu) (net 6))
 (segment (start 123.698 112.014) (end 123.952 111.76) (width 0.25) (layer B.Cu) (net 6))
 (segment (start 128.238 108.934) (end 128.016 108.712) (width 0.25) (layer B.Cu) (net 6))
 (via (at 128.016 108.712) (size 0.6) (drill 0.4) (layers F.Cu B.Cu) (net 6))
 (segment (start 109.093 108.839) (end 109.093 97.282) (width 0.25) (layer B.Cu) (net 6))
 (segment (start 109.093 97.282) (end 112.649 93.726) (width 0.25) (layer B.Cu) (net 6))
 (segment (start 125.476 119.888) (end 127.476 119.888) (width 0.25) (layer B.Cu) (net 6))
 (segment (start 128.016 113.4491) (end 128.016 116.586) (width 0.25) (layer F.Cu) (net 6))
 (segment (start 127.476 117.126) (end 127.476 119.888) (width 0.25) (layer B.Cu) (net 6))
 (segment (start 128.016 116.586) (end 127.476 117.126) (width 0.25) (layer B.Cu) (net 6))
 (via (at 128.016 116.586) (size 0.6) (drill 0.4) (layers F.Cu B.Cu) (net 6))
 (segment (start 106.807 108.839) (end 106.807 117.221) (width 0.25) (layer B.Cu) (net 6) (status 10))
 (segment (start 106.807 117.221) (end 107.061 117.475) (width 0.25) (layer B.Cu) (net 6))
 (segment (start 128.016 108.712) (end 128.016 113.4491) (width 0.25) (layer F.Cu) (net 6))
 (segment (start 116.84 108.372) (end 116.84 112.014) (width 0.25) (layer F.Cu) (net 6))
 (via (at 116.84 112.014) (size 0.6) (drill 0.4) (layers F.Cu B.Cu) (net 6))
 (segment (start 106.807 108.839) (end 109.093 108.839) (width 0.25) (layer B.Cu) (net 6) (status 10))
 (segment (start 109.093 108.839) (end 112.268 112.014) (width 0.25) (layer B.Cu) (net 6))
 (segment (start 112.268 112.014) (end 116.84 112.014) (width 0.25) (layer B.Cu) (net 6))
 (segment (start 107.315 117.221) (end 107.061 117.475) (width 0.25) (layer B.Cu) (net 6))
 (segment (start 107.188 108.458) (end 106.807 108.839) (width 0.25) (layer B.Cu) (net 6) (status 30))
 (segment (start 116.84 108.372) (end 116.84 101.992) (width 0.25) (layer F.Cu) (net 6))
 (segment (start 144.526 119.094) (end 143.732 119.888) (width 0.25) (layer B.Cu) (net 6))
 (segment (start 128.016 116.586) (end 132.842 116.586) (width 0.25) (layer B.Cu) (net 6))
 (segment (start 144.526 118.364) (end 144.526 119.094) (width 0.25) (layer B.Cu) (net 6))
 (segment (start 132.842 116.586) (end 134.62 118.364) (width 0.25) (layer B.Cu) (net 6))
 (segment (start 134.62 118.364) (end 144.526 118.364) (width 0.25) (layer B.Cu) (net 6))
 (segment (start 106.553 92.456) (end 106.553 101.854) (width 0.25) (layer F.Cu) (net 42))
 (segment (start 106.553 101.854) (end 106.807 102.108) (width 0.25) (layer F.Cu) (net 42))
 (segment (start 124.6124 113.4491) (end 126.3142 113.4491) (width 0.25) (layer F.Cu) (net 42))
 (segment (start 115.12 108.372) (end 115.12 112.464) (width 0.25) (layer F.Cu) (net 42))
 (segment (start 116.1051 113.4491) (end 124.6124 113.4491) (width 0.25) (layer F.Cu) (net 42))
 (segment (start 115.12 112.464) (end 116.1051 113.4491) (width 0.25) (layer F.Cu) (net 42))
 (segment (start 113.4 108.372) (end 115.12 108.372) (width 0.25) (layer F.Cu) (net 42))
 (segment (start 113.4 108.372) (end 113.4 117.083) (width 0.25) (layer F.Cu) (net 42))
 (segment (start 113.4 117.083) (end 113.792 117.475) (width 0.25) (layer F.Cu) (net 42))
 (segment (start 106.807 102.108) (end 106.807 102.287) (width 0.25) (layer F.Cu) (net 42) (status 30))
 (segment (start 106.807 102.287) (end 113.4 108.372) (width 0.25) (layer F.Cu) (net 42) (status 10))
 (segment (start 145.732 119.888) (end 145.732 118.428) (width 0.25) (layer B.Cu) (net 5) (status 1000000))
 (segment (start 145.732 118.428) (end 152.4476 111.7124) (width 0.25) (layer B.Cu) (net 5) (status 1000000))
 (segment (start 152.4476 111.7124) (end 164.2872 111.7124) (width 0.25) (layer B.Cu) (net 5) (status 1000000))
 (segment (start 129.7178 113.4491) (end 129.7178 118.7958) (width 0.25) (layer F.Cu) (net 7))
 (segment (start 129.7178 118.7958) (end 130.81 119.888) (width 0.25) (layer F.Cu) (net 7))
 (segment (start 130.9878 119.7102) (end 130.81 119.888) (width 0.25) (layer F.Cu) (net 7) (status 30))
 (segment (start 130.81 119.888) (end 132.81 119.888) (width 0.25) (layer F.Cu) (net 7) (status 30))
 (segment (start 132.81 119.888) (end 142.24 119.888) (width 0.25) (layer F.Cu) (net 7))
 (segment (start 163.580094 112.9284) (end 164.2872 112.9284) (width 0.25) (layer B.Cu) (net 4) (status 1000000))
 (segment (start 148.406999 119.213001) (end 148.406999 118.164591) (width 0.25) (layer B.Cu) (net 4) (status 1000000))
 (segment (start 147.732 119.888) (end 148.406999 119.213001) (width 0.25) (layer B.Cu) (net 4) (status 1000000))
 (segment (start 148.406999 118.164591) (end 153.64319 112.9284) (width 0.25) (layer B.Cu) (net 4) (status 1000000))
 (segment (start 153.64319 112.9284) (end 163.580094 112.9284) (width 0.25) (layer B.Cu) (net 4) (status 1000000))
 (segment (start 163.580094 114.1444) (end 164.2872 114.1444) (width 0.25) (layer B.Cu) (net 3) (status 1000000))
 (segment (start 150.406999 118.857999) (end 155.120598 114.1444) (width 0.25) (layer B.Cu) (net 3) (status 1000000))
 (segment (start 155.120598 114.1444) (end 163.580094 114.1444) (width 0.25) (layer B.Cu) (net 3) (status 1000000))
 (segment (start 149.732 119.888) (end 150.406999 119.213001) (width 0.25) (layer B.Cu) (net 3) (status 1000000))
 (segment (start 150.406999 119.213001) (end 150.406999 118.857999) (width 0.25) (layer B.Cu) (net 3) (status 1000000)))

